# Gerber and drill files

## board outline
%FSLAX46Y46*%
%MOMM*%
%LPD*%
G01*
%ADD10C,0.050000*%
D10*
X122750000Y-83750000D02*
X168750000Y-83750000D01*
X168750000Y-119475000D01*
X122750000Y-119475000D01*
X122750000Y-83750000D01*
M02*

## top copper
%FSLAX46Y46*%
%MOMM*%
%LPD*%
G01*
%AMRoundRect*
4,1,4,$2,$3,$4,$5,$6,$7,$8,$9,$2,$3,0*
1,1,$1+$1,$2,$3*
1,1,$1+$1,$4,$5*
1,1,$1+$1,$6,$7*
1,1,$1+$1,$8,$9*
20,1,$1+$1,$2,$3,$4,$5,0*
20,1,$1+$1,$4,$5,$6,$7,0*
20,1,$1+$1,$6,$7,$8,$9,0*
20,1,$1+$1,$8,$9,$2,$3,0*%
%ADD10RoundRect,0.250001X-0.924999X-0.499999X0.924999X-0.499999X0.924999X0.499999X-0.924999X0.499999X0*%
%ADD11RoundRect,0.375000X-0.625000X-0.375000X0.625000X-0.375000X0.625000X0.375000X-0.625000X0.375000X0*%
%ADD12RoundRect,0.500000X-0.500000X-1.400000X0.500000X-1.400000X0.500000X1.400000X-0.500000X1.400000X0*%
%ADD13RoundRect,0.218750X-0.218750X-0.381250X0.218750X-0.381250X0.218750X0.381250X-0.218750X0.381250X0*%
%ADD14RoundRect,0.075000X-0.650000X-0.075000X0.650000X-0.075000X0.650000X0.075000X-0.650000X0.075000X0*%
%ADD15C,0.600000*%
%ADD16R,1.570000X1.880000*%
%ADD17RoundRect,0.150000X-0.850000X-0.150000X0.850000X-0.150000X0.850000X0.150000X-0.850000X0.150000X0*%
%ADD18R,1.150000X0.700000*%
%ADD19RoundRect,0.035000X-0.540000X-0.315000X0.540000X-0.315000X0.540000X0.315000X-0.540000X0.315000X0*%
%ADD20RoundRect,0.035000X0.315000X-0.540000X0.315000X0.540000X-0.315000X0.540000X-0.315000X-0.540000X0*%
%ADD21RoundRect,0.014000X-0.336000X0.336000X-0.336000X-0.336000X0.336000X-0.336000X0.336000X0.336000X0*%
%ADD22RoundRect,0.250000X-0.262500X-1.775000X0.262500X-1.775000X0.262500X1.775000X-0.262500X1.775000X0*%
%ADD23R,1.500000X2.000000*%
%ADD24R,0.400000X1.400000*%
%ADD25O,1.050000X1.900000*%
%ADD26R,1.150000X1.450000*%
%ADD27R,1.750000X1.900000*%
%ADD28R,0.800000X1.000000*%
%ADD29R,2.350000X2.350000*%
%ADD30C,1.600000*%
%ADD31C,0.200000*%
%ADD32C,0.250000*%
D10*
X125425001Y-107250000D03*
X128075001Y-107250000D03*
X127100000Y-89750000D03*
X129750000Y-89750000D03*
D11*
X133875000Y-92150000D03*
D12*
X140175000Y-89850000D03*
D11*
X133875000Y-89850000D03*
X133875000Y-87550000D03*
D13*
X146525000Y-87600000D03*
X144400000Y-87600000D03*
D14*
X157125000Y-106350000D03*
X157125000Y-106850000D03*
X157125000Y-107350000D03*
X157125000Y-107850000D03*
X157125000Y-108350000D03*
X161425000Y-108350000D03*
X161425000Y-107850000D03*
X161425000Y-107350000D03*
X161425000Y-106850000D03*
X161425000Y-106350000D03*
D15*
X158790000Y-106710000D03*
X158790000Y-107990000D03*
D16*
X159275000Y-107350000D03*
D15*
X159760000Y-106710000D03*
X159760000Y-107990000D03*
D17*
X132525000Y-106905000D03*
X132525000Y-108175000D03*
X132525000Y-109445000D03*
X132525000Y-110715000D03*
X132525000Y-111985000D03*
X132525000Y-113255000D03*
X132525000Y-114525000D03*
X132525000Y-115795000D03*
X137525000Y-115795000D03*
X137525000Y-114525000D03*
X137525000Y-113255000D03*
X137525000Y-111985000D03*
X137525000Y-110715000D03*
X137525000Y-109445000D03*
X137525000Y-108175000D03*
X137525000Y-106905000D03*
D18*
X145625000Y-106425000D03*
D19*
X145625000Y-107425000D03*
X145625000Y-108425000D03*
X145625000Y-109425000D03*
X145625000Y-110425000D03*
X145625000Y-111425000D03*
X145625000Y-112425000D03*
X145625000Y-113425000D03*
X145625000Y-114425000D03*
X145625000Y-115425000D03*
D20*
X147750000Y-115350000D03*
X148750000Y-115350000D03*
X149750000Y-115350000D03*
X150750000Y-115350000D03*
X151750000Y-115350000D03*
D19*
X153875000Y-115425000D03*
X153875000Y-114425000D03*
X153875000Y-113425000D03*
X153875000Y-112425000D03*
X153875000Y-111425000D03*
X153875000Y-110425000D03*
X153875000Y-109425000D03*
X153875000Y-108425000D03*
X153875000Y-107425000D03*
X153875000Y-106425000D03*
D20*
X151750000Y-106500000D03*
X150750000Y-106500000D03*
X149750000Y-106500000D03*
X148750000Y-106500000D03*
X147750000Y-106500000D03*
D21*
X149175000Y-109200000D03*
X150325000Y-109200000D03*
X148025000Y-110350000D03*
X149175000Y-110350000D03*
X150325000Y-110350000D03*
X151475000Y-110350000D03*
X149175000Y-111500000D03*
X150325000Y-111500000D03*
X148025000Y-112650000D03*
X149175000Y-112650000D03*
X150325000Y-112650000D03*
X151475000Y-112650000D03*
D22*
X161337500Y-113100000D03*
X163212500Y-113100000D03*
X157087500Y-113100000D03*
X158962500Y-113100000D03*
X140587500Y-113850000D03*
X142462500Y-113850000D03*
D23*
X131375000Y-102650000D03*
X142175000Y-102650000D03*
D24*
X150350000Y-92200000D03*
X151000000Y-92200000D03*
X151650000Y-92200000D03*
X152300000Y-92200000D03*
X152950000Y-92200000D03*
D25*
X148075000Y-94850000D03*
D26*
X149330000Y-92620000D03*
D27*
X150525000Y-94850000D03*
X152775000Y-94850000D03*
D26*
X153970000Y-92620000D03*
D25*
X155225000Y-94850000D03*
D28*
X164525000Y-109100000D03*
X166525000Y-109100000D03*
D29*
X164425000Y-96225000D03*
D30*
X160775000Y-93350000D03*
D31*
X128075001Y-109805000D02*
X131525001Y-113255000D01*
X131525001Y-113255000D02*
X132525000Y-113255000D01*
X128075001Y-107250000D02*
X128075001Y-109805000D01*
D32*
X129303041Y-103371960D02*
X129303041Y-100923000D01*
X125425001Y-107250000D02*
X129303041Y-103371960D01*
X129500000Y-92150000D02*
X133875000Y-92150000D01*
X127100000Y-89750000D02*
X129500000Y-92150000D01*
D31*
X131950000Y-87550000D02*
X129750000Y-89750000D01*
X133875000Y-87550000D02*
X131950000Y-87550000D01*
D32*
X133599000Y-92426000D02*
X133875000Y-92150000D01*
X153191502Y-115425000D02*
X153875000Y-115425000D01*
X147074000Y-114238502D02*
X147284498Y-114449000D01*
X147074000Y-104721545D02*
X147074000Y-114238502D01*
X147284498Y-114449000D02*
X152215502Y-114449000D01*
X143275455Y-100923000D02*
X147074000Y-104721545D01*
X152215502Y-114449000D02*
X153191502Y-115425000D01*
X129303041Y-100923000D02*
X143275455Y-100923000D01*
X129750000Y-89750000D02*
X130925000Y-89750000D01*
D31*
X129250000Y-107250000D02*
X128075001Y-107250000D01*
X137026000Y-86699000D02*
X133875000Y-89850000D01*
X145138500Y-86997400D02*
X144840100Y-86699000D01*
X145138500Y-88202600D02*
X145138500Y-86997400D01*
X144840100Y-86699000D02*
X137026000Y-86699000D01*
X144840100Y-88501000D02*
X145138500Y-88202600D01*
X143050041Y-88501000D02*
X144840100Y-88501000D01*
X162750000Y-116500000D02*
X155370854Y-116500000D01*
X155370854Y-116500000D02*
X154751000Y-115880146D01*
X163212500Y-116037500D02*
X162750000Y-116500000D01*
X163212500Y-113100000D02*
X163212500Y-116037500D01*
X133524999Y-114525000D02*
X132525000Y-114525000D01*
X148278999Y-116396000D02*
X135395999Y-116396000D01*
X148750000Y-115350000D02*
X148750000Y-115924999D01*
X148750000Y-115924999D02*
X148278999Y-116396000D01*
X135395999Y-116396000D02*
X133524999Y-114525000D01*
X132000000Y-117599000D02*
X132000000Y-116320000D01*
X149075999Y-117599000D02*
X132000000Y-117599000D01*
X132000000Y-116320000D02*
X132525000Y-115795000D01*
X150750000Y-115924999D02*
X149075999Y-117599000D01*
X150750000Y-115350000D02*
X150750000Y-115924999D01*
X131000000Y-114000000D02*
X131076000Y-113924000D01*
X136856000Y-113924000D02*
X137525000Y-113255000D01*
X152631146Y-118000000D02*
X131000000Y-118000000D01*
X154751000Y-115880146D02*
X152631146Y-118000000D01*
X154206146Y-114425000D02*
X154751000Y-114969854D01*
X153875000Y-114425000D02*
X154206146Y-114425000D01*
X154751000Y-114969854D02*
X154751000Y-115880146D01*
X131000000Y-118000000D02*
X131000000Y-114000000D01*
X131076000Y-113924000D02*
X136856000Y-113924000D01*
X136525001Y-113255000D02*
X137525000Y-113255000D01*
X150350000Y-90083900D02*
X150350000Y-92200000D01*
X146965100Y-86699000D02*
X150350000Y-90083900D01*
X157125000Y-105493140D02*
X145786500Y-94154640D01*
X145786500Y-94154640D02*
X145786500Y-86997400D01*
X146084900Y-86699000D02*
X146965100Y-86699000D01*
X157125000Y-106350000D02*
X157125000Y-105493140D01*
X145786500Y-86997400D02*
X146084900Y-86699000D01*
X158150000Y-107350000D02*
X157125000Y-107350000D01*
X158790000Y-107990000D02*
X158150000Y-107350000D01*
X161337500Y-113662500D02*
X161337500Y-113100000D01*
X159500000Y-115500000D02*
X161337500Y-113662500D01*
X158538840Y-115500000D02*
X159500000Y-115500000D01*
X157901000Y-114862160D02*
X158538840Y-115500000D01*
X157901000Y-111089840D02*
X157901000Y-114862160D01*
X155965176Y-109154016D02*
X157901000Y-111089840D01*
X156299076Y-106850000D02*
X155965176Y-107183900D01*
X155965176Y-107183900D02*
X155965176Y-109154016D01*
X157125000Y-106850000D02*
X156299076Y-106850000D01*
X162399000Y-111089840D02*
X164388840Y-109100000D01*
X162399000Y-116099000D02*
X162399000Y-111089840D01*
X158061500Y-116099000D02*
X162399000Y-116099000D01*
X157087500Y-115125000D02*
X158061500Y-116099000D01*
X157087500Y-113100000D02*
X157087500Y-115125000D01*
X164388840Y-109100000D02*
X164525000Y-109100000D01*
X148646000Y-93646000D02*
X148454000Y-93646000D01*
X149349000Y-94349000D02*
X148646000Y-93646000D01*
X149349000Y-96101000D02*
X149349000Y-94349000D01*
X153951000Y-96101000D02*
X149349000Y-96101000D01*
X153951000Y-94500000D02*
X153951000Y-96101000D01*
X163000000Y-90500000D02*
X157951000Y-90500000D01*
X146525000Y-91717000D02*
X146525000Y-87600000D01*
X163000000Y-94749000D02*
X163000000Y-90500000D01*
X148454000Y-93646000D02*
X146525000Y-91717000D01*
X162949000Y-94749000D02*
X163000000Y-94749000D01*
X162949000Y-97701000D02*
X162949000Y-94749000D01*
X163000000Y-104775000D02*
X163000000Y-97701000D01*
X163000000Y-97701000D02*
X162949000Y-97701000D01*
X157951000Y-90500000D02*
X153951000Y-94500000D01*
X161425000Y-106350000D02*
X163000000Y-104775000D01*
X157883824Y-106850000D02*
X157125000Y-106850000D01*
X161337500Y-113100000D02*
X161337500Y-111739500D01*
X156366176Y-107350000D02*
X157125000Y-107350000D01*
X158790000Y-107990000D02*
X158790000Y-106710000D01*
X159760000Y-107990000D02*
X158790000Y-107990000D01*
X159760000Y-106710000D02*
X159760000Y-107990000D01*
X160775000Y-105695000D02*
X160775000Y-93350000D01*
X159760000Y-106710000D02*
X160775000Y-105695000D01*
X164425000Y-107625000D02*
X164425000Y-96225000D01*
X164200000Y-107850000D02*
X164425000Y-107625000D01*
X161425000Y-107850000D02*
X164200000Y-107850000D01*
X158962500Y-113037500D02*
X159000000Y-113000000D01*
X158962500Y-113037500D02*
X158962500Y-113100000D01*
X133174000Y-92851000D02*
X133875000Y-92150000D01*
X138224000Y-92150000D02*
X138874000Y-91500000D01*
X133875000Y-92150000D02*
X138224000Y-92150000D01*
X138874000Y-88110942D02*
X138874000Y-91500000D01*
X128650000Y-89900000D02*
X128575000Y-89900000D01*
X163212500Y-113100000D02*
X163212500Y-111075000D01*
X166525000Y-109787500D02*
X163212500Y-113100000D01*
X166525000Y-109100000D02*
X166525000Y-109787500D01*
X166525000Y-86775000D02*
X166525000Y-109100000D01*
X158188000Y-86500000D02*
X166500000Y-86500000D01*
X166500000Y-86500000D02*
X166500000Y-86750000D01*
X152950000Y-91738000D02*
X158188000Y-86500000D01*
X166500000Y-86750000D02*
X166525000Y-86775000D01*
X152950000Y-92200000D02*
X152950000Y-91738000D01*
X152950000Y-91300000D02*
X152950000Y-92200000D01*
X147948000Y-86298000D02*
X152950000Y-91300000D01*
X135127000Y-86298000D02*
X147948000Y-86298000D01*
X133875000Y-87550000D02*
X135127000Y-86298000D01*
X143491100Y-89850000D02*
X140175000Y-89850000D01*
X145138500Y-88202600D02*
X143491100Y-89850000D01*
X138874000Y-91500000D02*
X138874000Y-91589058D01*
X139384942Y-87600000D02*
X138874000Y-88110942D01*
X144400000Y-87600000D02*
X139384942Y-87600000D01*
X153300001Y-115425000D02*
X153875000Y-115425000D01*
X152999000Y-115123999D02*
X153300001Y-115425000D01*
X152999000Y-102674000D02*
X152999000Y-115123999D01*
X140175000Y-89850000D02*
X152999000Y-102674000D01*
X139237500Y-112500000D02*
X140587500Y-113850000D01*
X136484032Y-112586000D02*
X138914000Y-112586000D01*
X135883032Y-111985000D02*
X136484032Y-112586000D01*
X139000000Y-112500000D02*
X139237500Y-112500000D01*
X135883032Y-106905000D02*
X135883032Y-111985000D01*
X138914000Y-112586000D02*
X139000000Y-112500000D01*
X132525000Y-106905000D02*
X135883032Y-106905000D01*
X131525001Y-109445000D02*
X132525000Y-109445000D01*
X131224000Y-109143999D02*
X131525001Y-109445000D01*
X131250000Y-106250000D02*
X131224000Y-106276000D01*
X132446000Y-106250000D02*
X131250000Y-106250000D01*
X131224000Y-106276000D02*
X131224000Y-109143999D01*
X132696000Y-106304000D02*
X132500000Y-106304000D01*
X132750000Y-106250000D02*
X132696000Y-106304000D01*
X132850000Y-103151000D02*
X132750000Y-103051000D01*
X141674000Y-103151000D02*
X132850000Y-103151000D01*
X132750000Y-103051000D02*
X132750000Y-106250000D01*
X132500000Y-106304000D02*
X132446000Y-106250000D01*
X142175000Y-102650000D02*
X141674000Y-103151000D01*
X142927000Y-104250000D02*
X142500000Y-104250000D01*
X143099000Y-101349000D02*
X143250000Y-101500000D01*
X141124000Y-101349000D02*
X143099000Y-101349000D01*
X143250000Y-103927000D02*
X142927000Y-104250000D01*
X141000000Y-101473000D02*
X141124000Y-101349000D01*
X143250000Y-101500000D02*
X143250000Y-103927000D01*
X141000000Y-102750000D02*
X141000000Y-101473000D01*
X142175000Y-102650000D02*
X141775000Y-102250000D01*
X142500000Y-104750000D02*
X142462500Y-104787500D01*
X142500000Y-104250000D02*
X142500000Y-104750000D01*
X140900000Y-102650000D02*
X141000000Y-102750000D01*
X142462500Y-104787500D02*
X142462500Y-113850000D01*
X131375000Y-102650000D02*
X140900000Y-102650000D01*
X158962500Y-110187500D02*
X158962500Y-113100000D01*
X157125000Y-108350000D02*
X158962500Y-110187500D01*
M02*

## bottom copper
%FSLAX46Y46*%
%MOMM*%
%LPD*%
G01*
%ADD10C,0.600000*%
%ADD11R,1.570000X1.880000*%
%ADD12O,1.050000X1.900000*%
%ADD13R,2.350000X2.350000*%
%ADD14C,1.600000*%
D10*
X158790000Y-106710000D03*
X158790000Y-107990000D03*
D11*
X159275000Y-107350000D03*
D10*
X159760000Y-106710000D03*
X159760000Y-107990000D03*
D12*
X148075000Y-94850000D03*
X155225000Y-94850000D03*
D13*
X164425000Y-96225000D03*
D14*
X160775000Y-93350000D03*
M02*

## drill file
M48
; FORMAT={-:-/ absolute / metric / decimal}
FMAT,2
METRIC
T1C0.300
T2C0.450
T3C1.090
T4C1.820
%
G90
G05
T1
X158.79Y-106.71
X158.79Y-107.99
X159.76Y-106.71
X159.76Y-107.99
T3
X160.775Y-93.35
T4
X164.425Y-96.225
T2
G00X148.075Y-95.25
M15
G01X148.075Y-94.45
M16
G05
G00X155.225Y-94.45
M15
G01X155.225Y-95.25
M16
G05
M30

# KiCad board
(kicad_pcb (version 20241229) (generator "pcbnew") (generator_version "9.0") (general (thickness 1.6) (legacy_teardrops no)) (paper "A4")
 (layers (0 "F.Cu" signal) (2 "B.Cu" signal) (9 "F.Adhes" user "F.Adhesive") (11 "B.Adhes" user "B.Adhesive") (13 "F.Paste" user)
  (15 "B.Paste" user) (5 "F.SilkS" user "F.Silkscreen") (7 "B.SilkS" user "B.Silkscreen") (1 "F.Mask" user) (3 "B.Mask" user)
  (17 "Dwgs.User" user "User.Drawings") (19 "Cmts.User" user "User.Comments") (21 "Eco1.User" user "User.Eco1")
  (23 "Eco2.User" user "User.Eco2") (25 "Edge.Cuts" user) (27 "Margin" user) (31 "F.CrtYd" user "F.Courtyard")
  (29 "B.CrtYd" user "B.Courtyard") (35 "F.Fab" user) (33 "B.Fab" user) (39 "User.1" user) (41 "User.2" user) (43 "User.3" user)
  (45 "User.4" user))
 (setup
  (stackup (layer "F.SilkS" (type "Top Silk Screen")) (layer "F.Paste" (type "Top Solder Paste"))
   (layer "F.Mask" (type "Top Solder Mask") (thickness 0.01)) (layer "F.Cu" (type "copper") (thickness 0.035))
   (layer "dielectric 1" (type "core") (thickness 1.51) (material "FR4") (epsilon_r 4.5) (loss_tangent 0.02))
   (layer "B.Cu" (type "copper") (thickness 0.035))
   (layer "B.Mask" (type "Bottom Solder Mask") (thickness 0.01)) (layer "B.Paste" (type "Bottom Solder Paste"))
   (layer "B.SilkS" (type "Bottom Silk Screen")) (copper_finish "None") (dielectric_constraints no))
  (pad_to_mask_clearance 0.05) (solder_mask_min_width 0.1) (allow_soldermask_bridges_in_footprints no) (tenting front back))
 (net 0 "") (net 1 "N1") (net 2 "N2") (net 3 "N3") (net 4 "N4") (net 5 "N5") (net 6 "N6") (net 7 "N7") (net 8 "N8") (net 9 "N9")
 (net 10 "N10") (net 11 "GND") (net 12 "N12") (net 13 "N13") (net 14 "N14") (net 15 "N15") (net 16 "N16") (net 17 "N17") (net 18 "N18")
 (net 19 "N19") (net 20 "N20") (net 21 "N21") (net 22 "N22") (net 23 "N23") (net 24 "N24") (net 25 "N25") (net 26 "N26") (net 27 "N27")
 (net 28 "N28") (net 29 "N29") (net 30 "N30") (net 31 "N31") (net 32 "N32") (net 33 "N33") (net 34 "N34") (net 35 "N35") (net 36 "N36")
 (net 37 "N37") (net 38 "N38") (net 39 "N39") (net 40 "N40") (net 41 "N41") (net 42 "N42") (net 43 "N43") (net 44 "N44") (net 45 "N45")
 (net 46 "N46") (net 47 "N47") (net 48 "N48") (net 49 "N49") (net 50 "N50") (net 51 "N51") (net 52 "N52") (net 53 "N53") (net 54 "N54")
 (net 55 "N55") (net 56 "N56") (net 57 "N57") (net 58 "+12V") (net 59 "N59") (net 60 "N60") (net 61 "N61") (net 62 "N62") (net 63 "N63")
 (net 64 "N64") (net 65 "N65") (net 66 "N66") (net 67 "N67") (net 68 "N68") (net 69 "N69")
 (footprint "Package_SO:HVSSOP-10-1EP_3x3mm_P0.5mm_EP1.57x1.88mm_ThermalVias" (layer "F.Cu") (at 159.275 107.35)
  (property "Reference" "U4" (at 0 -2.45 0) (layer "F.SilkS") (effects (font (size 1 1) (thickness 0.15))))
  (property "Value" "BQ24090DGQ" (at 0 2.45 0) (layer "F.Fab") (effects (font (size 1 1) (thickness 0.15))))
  (pad "" smd roundrect (at -0.39 -0.47) (size 0.63 0.76) (layers "F.Paste") (roundrect_rratio 0.25))
  (pad "" smd roundrect (at -0.39 0.47) (size 0.63 0.76) (layers "F.Paste") (roundrect_rratio 0.25))
  (pad "" smd roundrect (at 0.39 -0.47) (size 0.63 0.76) (layers "F.Paste") (roundrect_rratio 0.25))
  (pad "" smd roundrect (at 0.39 0.47) (size 0.63 0.76) (layers "F.Paste") (roundrect_rratio 0.25))
  (pad "1" smd roundrect (at -2.15 -1) (size 1.45 0.3) (layers "F.Cu" "F.Mask" "F.Paste") (roundrect_rratio 0.25) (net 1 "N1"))
  (pad "2" smd roundrect (at -2.15 -0.5) (size 1.45 0.3) (layers "F.Cu" "F.Mask" "F.Paste") (roundrect_rratio 0.25) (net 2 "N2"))
  (pad "3" smd roundrect (at -2.15 0) (size 1.45 0.3) (layers "F.Cu" "F.Mask" "F.Paste") (roundrect_rratio 0.25) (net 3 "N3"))
  (pad "4" smd roundrect (at -2.15 0.5) (size 1.45 0.3) (layers "F.Cu" "F.Mask" "F.Paste") (roundrect_rratio 0.25) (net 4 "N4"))
  (pad "5" smd roundrect (at -2.15 1) (size 1.45 0.3) (layers "F.Cu" "F.Mask" "F.Paste") (roundrect_rratio 0.25) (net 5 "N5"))
  (pad "6" smd roundrect (at 2.15 1) (size 1.45 0.3) (layers "F.Cu" "F.Mask" "F.Paste") (roundrect_rratio 0.25) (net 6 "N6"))
  (pad "7" smd roundrect (at 2.15 0.5) (size 1.45 0.3) (layers "F.Cu" "F.Mask" "F.Paste") (roundrect_rratio 0.25) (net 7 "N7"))
  (pad "8" smd roundrect (at 2.15 0) (size 1.45 0.3) (layers "F.Cu" "F.Mask" "F.Paste") (roundrect_rratio 0.25) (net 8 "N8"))
  (pad "9" smd roundrect (at 2.15 -0.5) (size 1.45 0.3) (layers "F.Cu" "F.Mask" "F.Paste") (roundrect_rratio 0.25) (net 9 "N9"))
  (pad "10" smd roundrect (at 2.15 -1) (size 1.45 0.3) (layers "F.Cu" "F.Mask" "F.Paste") (roundrect_rratio 0.25) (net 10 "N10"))
  (pad "11" thru_hole circle (at -0.485 -0.64) (size 0.6 0.6) (drill 0.3) (layers "*.Cu") (remove_unused_layers no) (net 3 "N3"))
  (pad "11" thru_hole circle (at -0.485 0.64) (size 0.6 0.6) (drill 0.3) (layers "*.Cu") (remove_unused_layers no) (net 3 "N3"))
  (pad "11" smd rect (at 0 0) (size 1.57 1.88) (layers "F.Cu" "F.Mask") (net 3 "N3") (zone_connect 2))
  (pad "11" smd rect (at 0 0) (size 1.57 1.88) (layers "B.Cu") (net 3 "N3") (zone_connect 2))
  (pad "11" thru_hole circle (at 0.485 -0.64) (size 0.6 0.6) (drill 0.3) (layers "*.Cu") (remove_unused_layers no) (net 3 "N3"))
  (pad "11" thru_hole circle (at 0.485 0.64) (size 0.6 0.6) (drill 0.3) (layers "*.Cu") (remove_unused_layers no) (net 3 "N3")))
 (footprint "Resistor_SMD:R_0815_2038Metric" (layer "F.Cu") (at 162.275 113.1)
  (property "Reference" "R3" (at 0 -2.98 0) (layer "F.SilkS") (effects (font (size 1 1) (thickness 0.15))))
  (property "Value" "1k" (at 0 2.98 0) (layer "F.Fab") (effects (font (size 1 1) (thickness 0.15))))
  (pad "1" smd roundrect (at -0.9375 0) (size 1.025 4.05) (layers "F.Cu" "F.Mask" "F.Paste") (roundrect_rratio 0.243902) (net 2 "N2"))
  (pad "2" smd roundrect (at 0.9375 0) (size 1.025 4.05) (layers "F.Cu" "F.Mask" "F.Paste") (roundrect_rratio 0.243902) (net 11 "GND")))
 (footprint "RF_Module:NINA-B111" (layer "F.Cu") (at 149.75 110.925)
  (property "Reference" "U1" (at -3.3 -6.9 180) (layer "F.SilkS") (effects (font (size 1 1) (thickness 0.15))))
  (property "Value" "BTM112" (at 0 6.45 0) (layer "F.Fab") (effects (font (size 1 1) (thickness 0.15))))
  (pad "1" smd rect (at -4.125 -4.5) (size 1.15 0.7) (layers "F.Cu" "F.Mask" "F.Paste") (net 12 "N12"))
  (pad "2" smd roundrect (at -4.125 -3.5) (size 1.15 0.7) (layers "F.Cu" "F.Mask" "F.Paste") (roundrect_rratio 0.05) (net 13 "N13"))
  (pad "3" smd roundrect (at -4.125 -2.5) (size 1.15 0.7) (layers "F.Cu" "F.Mask" "F.Paste") (roundrect_rratio 0.05) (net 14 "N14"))
  (pad "4" smd roundrect (at -4.125 -1.5) (size 1.15 0.7) (layers "F.Cu" "F.Mask" "F.Paste") (roundrect_rratio 0.05) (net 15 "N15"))
  (pad "5" smd roundrect (at -4.125 -0.5) (size 1.15 0.7) (layers "F.Cu" "F.Mask" "F.Paste") (roundrect_rratio 0.05) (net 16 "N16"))
  (pad "6" smd roundrect (at -4.125 0.5) (size 1.15 0.7) (layers "F.Cu" "F.Mask" "F.Paste") (roundrect_rratio 0.05) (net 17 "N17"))
  (pad "7" smd roundrect (at -4.125 1.5) (size 1.15 0.7) (layers "F.Cu" "F.Mask" "F.Paste") (roundrect_rratio 0.05) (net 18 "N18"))
  (pad "8" smd roundrect (at -4.125 2.5) (size 1.15 0.7) (layers "F.Cu" "F.Mask" "F.Paste") (roundrect_rratio 0.05) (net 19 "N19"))
  (pad "9" smd roundrect (at -4.125 3.5) (size 1.15 0.7) (layers "F.Cu" "F.Mask" "F.Paste") (roundrect_rratio 0.05) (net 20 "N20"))
  (pad "10" smd roundrect (at -4.125 4.5) (size 1.15 0.7) (layers "F.Cu" "F.Mask" "F.Paste") (roundrect_rratio 0.05) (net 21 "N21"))
  (pad "11" smd roundrect (at -2 4.425 90) (size 1.15 0.7) (layers "F.Cu" "F.Mask" "F.Paste") (roundrect_rratio 0.05) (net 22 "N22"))
  (pad "12" smd roundrect (at -1 4.425 90) (size 1.15 0.7) (layers "F.Cu" "F.Mask" "F.Paste") (roundrect_rratio 0.05) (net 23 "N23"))
  (pad "13" smd roundrect (at 0 4.425 90) (size 1.15 0.7) (layers "F.Cu" "F.Mask" "F.Paste") (roundrect_rratio 0.05) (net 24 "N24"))
  (pad "14" smd roundrect (at 1 4.425 90) (size 1.15 0.7) (layers "F.Cu" "F.Mask" "F.Paste") (roundrect_rratio 0.05) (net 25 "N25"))
  (pad "15" smd roundrect (at 2 4.425 90) (size 1.15 0.7) (layers "F.Cu" "F.Mask" "F.Paste") (roundrect_rratio 0.05) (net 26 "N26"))
  (pad "16" smd roundrect (at 4.125 4.5) (size 1.15 0.7) (layers "F.Cu" "F.Mask" "F.Paste") (roundrect_rratio 0.05) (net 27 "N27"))
  (pad "17" smd roundrect (at 4.125 3.5) (size 1.15 0.7) (layers "F.Cu" "F.Mask" "F.Paste") (roundrect_rratio 0.05) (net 11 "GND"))
  (pad "18" smd roundrect (at 4.125 2.5) (size 1.15 0.7) (layers "F.Cu" "F.Mask" "F.Paste") (roundrect_rratio 0.05) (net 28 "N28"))
  (pad "19" smd roundrect (at 4.125 1.5) (size 1.15 0.7) (layers "F.Cu" "F.Mask" "F.Paste") (roundrect_rratio 0.05) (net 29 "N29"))
  (pad "20" smd roundrect (at 4.125 0.5) (size 1.15 0.7) (layers "F.Cu" "F.Mask" "F.Paste") (roundrect_rratio 0.05) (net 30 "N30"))
  (pad "21" smd roundrect (at 4.125 -0.5) (size 1.15 0.7) (layers "F.Cu" "F.Mask" "F.Paste") (roundrect_rratio 0.05) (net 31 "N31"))
  (pad "22" smd roundrect (at 4.125 -1.5) (size 1.15 0.7) (layers "F.Cu" "F.Mask" "F.Paste") (roundrect_rratio 0.05) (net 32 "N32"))
  (pad "23" smd roundrect (at 4.125 -2.5) (size 1.15 0.7) (layers "F.Cu" "F.Mask" "F.Paste") (roundrect_rratio 0.05) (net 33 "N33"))
  (pad "24" smd roundrect (at 4.125 -3.5) (size 1.15 0.7) (layers "F.Cu" "F.Mask" "F.Paste") (roundrect_rratio 0.05) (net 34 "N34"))
  (pad "25" smd roundrect (at 4.125 -4.5) (size 1.15 0.7) (layers "F.Cu" "F.Mask" "F.Paste") (roundrect_rratio 0.05) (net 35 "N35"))
  (pad "26" smd roundrect (at 2 -4.425 90) (size 1.15 0.7) (layers "F.Cu" "F.Mask" "F.Paste") (roundrect_rratio 0.05) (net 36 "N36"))
  (pad "27" smd roundrect (at 1 -4.425 90) (size 1.15 0.7) (layers "F.Cu" "F.Mask" "F.Paste") (roundrect_rratio 0.05) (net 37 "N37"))
  (pad "28" smd roundrect (at 0 -4.425 90) (size 1.15 0.7) (layers "F.Cu" "F.Mask" "F.Paste") (roundrect_rratio 0.05) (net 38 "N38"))
  (pad "29" smd roundrect (at -1 -4.425 90) (size 1.15 0.7) (layers "F.Cu" "F.Mask" "F.Paste") (roundrect_rratio 0.05) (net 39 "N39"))
  (pad "30" smd roundrect (at -2 -4.425 90) (size 1.15 0.7) (layers "F.Cu" "F.Mask" "F.Paste") (roundrect_rratio 0.05) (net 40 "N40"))
  (pad "31" smd roundrect (at -0.575 -1.725 270) (size 0.7 0.7) (layers "F.Cu" "F.Mask" "F.Paste") (roundrect_rratio 0.02) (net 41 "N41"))
  (pad "32" smd roundrect (at 0.575 -1.725 270) (size 0.7 0.7) (layers "F.Cu" "F.Mask" "F.Paste") (roundrect_rratio 0.02) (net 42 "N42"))
  (pad "33" smd roundrect (at -1.725 -0.575 270) (size 0.7 0.7) (layers "F.Cu" "F.Mask" "F.Paste") (roundrect_rratio 0.02) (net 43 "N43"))
  (pad "34" smd roundrect (at -0.575 -0.575 270) (size 0.7 0.7) (layers "F.Cu" "F.Mask" "F.Paste") (roundrect_rratio 0.02) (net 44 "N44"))
  (pad "35" smd roundrect (at 0.575 -0.575 270) (size 0.7 0.7) (layers "F.Cu" "F.Mask" "F.Paste") (roundrect_rratio 0.02))
  (pad "36" smd roundrect (at 1.725 -0.575 270) (size 0.7 0.7) (layers "F.Cu" "F.Mask" "F.Paste") (roundrect_rratio 0.02))
  (pad "37" smd roundrect (at -0.575 0.575 270) (size 0.7 0.7) (layers "F.Cu" "F.Mask" "F.Paste") (roundrect_rratio 0.02))
  (pad "38" smd roundrect (at 0.575 0.575 270) (size 0.7 0.7) (layers "F.Cu" "F.Mask" "F.Paste") (roundrect_rratio 0.02))
  (pad "39" smd roundrect (at -1.725 1.725 270) (size 0.7 0.7) (layers "F.Cu" "F.Mask" "F.Paste") (roundrect_rratio 0.02))
  (pad "40" smd roundrect (at -0.575 1.725 270) (size 0.7 0.7) (layers "F.Cu" "F.Mask" "F.Paste") (roundrect_rratio 0.02))
  (pad "41" smd roundrect (at 0.575 1.725 270) (size 0.7 0.7) (layers "F.Cu" "F.Mask" "F.Paste") (roundrect_rratio 0.02))
  (pad "42" smd roundrect (at 1.725 1.725 270) (size 0.7 0.7) (layers "F.Cu" "F.Mask" "F.Paste") (roundrect_rratio 0.02))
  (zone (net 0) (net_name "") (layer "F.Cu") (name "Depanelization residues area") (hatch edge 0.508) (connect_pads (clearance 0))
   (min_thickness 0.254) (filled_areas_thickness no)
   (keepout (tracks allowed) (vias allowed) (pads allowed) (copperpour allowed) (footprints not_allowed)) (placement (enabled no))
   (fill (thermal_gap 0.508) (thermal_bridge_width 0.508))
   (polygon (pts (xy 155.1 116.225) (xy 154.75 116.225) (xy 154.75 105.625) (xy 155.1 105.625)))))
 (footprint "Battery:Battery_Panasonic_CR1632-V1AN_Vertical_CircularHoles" (layer "F.Cu") (at 164.425 96.225 90)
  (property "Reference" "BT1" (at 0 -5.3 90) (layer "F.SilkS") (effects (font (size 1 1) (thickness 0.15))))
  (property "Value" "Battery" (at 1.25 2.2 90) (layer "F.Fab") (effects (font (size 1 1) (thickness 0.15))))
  (pad "1" thru_hole rect (at 0 0 180) (size 2.35 2.35) (drill 1.82) (layers "*.Cu" "*.Mask") (remove_unused_layers no) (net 7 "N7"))
  (pad "2" thru_hole circle (at 2.875 -3.65 90) (size 1.6 1.6) (drill 1.09) (layers "*.Cu" "*.Mask") (remove_unused_layers no) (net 3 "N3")))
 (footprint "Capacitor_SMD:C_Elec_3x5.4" (layer "F.Cu") (at 126.750001 107.25)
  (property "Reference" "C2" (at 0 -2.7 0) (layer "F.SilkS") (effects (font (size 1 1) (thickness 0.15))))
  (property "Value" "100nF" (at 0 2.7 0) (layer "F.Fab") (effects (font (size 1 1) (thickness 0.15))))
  (pad "1" smd roundrect (at -1.325 0) (size 2.35 1.5) (layers "F.Cu" "F.Mask" "F.Paste") (roundrect_rratio 0.166667) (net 27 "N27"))
  (pad "2" smd roundrect (at 1.325 0) (size 2.35 1.5) (layers "F.Cu" "F.Mask" "F.Paste") (roundrect_rratio 0.166667) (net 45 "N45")))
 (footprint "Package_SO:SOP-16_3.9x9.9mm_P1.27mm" (layer "F.Cu") (at 135.025 111.35)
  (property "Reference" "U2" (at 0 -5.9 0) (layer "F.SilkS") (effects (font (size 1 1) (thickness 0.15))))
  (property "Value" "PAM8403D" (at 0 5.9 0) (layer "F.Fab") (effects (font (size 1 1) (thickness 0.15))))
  (pad "1" smd roundrect (at -2.5 -4.445) (size 2 0.6) (layers "F.Cu" "F.Mask" "F.Paste") (roundrect_rratio 0.25) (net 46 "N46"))
  (pad "2" smd roundrect (at -2.5 -3.175) (size 2 0.6) (layers "F.Cu" "F.Mask" "F.Paste") (roundrect_rratio 0.25) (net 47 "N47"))
  (pad "3" smd roundrect (at -2.5 -1.905) (size 2 0.6) (layers "F.Cu" "F.Mask" "F.Paste") (roundrect_rratio 0.25) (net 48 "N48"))
  (pad "4" smd roundrect (at -2.5 -0.635) (size 2 0.6) (layers "F.Cu" "F.Mask" "F.Paste") (roundrect_rratio 0.25) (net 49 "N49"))
  (pad "5" smd roundrect (at -2.5 0.635) (size 2 0.6) (layers "F.Cu" "F.Mask" "F.Paste") (roundrect_rratio 0.25) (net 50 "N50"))
  (pad "6" smd roundrect (at -2.5 1.905) (size 2 0.6) (layers "F.Cu" "F.Mask" "F.Paste") (roundrect_rratio 0.25) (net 45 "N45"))
  (pad "7" smd roundrect (at -2.5 3.175) (size 2 0.6) (layers "F.Cu" "F.Mask" "F.Paste") (roundrect_rratio 0.25) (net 23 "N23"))
  (pad "8" smd roundrect (at -2.5 4.445) (size 2 0.6) (layers "F.Cu" "F.Mask" "F.Paste") (roundrect_rratio 0.25) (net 25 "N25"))
  (pad "9" smd roundrect (at 2.5 4.445) (size 2 0.6) (layers "F.Cu" "F.Mask" "F.Paste") (roundrect_rratio 0.25) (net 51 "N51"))
  (pad "10" smd roundrect (at 2.5 3.175) (size 2 0.6) (layers "F.Cu" "F.Mask" "F.Paste") (roundrect_rratio 0.25) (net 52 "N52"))
  (pad "11" smd roundrect (at 2.5 1.905) (size 2 0.6) (layers "F.Cu" "F.Mask" "F.Paste") (roundrect_rratio 0.25) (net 11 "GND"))
  (pad "12" smd roundrect (at 2.5 0.635) (size 2 0.6) (layers "F.Cu" "F.Mask" "F.Paste") (roundrect_rratio 0.25) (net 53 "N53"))
  (pad "13" smd roundrect (at 2.5 -0.635) (size 2 0.6) (layers "F.Cu" "F.Mask" "F.Paste") (roundrect_rratio 0.25) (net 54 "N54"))
  (pad "14" smd roundrect (at 2.5 -1.905) (size 2 0.6) (layers "F.Cu" "F.Mask" "F.Paste") (roundrect_rratio 0.25) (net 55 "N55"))
  (pad "15" smd roundrect (at 2.5 -3.175) (size 2 0.6) (layers "F.Cu" "F.Mask" "F.Paste") (roundrect_rratio 0.25) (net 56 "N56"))
  (pad "16" smd roundrect (at 2.5 -4.445) (size 2 0.6) (layers "F.Cu" "F.Mask" "F.Paste") (roundrect_rratio 0.25) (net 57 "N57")))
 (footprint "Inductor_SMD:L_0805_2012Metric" (layer "F.Cu") (at 145.4625 87.6)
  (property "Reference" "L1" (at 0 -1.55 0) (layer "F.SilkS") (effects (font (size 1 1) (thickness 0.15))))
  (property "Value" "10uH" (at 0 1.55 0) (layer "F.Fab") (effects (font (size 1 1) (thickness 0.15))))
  (pad "1" smd roundrect (at -1.0625 0) (size 0.875 1.2) (layers "F.Cu" "F.Mask" "F.Paste") (roundrect_rratio 0.25) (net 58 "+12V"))
  (pad "2" smd roundrect (at 1.0625 0) (size 0.875 1.2) (layers "F.Cu" "F.Mask" "F.Paste") (roundrect_rratio 0.25) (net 10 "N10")))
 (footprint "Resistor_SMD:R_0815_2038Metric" (layer "F.Cu") (at 141.525 113.85)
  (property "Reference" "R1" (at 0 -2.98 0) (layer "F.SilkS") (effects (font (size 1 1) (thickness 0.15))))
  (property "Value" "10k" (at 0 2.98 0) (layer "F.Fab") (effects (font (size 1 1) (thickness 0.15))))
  (pad "1" smd roundrect (at -0.9375 0) (size 1.025 4.05) (layers "F.Cu" "F.Mask" "F.Paste") (roundrect_rratio 0.243902) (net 46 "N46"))
  (pad "2" smd roundrect (at 0.9375 0) (size 1.025 4.05) (layers "F.Cu" "F.Mask" "F.Paste") (roundrect_rratio 0.243902) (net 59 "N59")))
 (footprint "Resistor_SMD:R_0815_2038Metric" (layer "F.Cu") (at 158.025 113.1)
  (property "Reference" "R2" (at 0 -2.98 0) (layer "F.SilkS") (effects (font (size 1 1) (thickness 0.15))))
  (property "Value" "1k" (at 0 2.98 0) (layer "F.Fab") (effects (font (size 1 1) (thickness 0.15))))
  (pad "1" smd roundrect (at -0.9375 0) (size 1.025 4.05) (layers "F.Cu" "F.Mask" "F.Paste") (roundrect_rratio 0.243902) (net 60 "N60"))
  (pad "2" smd roundrect (at 0.9375 0) (size 1.025 4.05) (layers "F.Cu" "F.Mask" "F.Paste") (roundrect_rratio 0.243902) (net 5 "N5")))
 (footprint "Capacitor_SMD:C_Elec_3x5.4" (layer "F.Cu") (at 128.425 89.75)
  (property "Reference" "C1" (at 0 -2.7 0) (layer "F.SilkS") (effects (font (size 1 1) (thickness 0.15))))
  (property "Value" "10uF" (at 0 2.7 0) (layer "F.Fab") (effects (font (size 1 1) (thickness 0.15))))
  (pad "1" smd roundrect (at -1.325 0) (size 2.35 1.5) (layers "F.Cu" "F.Mask" "F.Paste") (roundrect_rratio 0.166667) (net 58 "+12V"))
  (pad "2" smd roundrect (at 1.325 0) (size 2.35 1.5) (layers "F.Cu" "F.Mask" "F.Paste") (roundrect_rratio 0.166667) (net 11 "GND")))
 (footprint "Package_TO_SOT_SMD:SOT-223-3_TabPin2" (layer "F.Cu") (at 137.025 89.85)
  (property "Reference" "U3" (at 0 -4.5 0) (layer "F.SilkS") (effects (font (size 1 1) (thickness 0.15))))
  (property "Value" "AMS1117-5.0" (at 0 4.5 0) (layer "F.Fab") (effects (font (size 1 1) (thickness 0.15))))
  (pad "1" smd roundrect (at -3.15 -2.3) (size 2 1.5) (layers "F.Cu" "F.Mask" "F.Paste") (roundrect_rratio 0.25) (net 11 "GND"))
  (pad "2" smd roundrect (at -3.15 0) (size 2 1.5) (layers "F.Cu" "F.Mask" "F.Paste") (roundrect_rratio 0.25) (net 27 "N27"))
  (pad "2" smd roundrect (at 3.15 0) (size 2 3.8) (layers "F.Cu" "F.Mask" "F.Paste") (roundrect_rratio 0.25) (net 27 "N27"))
  (pad "3" smd roundrect (at -3.15 2.3) (size 2 1.5) (layers "F.Cu" "F.Mask" "F.Paste") (roundrect_rratio 0.25) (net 58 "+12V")))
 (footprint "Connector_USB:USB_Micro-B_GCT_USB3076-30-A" (layer "F.Cu") (at 151.65 93.65)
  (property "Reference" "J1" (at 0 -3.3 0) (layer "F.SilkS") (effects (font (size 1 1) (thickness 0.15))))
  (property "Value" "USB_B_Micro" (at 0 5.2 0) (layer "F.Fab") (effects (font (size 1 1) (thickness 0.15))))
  (pad "1" smd rect (at -1.3 -1.45) (size 0.4 1.4) (layers "F.Cu" "F.Mask" "F.Paste") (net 1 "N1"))
  (pad "2" smd rect (at -0.65 -1.45) (size 0.4 1.4) (layers "F.Cu" "F.Mask" "F.Paste") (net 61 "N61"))
  (pad "3" smd rect (at 0 -1.45) (size 0.4 1.4) (layers "F.Cu" "F.Mask" "F.Paste") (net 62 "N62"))
  (pad "4" smd rect (at 0.65 -1.45) (size 0.4 1.4) (layers "F.Cu" "F.Mask" "F.Paste") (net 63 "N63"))
  (pad "5" smd rect (at 1.3 -1.45) (size 0.4 1.4) (layers "F.Cu" "F.Mask" "F.Paste") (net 11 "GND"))
  (pad "6" thru_hole oval (at -3.575 1.2 180) (size 1.05 1.9) (drill oval 0.45 1.25) (layers "*.Cu" "*.Mask") (remove_unused_layers no)
   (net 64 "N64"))
  (pad "6" smd rect (at -2.32 -1.03) (size 1.15 1.45) (layers "F.Cu" "F.Mask" "F.Paste") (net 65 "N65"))
  (pad "6" smd rect (at -1.125 1.2) (size 1.75 1.9) (layers "F.Cu" "F.Mask" "F.Paste") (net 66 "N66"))
  (pad "6" smd rect (at 1.125 1.2) (size 1.75 1.9) (layers "F.Cu" "F.Mask" "F.Paste") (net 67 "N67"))
  (pad "6" smd rect (at 2.32 -1.03) (size 1.15 1.45) (layers "F.Cu" "F.Mask" "F.Paste") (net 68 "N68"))
  (pad "6" thru_hole oval (at 3.575 1.2) (size 1.05 1.9) (drill oval 0.45 1.25) (layers "*.Cu" "*.Mask") (remove_unused_layers no)
   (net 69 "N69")))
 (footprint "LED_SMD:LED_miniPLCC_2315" (layer "F.Cu") (at 165.525 109.1)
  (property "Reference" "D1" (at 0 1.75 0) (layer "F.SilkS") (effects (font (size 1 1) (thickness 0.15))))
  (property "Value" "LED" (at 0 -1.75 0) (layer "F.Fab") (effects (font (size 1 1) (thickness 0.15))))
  (pad "1" smd rect (at -1 0 180) (size 0.8 1) (layers "F.Cu" "F.Mask" "F.Paste") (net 60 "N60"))
  (pad "2" smd rect (at 1 0 180) (size 0.8 1) (layers "F.Cu" "F.Mask" "F.Paste") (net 11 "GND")))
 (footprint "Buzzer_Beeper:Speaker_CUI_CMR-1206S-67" (layer "F.Cu") (at 136.775 100.35)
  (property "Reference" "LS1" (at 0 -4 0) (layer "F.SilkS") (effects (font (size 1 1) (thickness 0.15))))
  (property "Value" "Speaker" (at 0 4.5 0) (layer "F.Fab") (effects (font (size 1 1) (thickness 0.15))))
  (pad "1" smd rect (at -5.4 2.3 180) (size 1.5 2) (layers "F.Cu" "F.Mask") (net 59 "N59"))
  (pad "2" smd rect (at 5.4 2.3 180) (size 1.5 2) (layers "F.Cu" "F.Mask") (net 48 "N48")))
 (gr_rect (start 122.75 83.75) (end 168.75 119.475) (stroke (width 0.05) (type default)) (fill no) (layer "Edge.Cuts"))
 (segment (start 156.366176 107.35) (end 157.125 107.35) (width 0.2) (layer "F.Cu") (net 3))
 (segment (start 158.15 107.35) (end 157.125 107.35) (width 0.2) (layer "F.Cu") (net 3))
 (segment (start 159.76 107.99) (end 158.79 107.99) (width 0.2) (layer "F.Cu") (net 3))
 (segment (start 160.775 105.695) (end 160.775 93.35) (width 0.2) (layer "F.Cu") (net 3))
 (segment (start 158.79 107.99) (end 158.79 106.71) (width 0.2) (layer "F.Cu") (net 3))
 (segment (start 158.79 107.99) (end 158.15 107.35) (width 0.2) (layer "F.Cu") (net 3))
 (segment (start 159.76 106.71) (end 160.775 105.695) (width 0.2) (layer "F.Cu") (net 3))
 (segment (start 159.76 106.71) (end 159.76 107.99) (width 0.2) (layer "F.Cu") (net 3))
 (segment (start 164.425 107.625) (end 164.425 96.225) (width 0.2) (layer "F.Cu") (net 7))
 (segment (start 164.2 107.85) (end 164.425 107.625) (width 0.2) (layer "F.Cu") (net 7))
 (segment (start 161.425 107.85) (end 164.2 107.85) (width 0.2) (layer "F.Cu") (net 7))
 (segment (start 144.4 87.6) (end 139.384942 87.6) (width 0.2) (layer "F.Cu") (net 58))
 (segment (start 129.5 92.15) (end 133.875 92.15) (width 0.25) (layer "F.Cu") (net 58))
 (segment (start 139.384942 87.6) (end 138.874 88.110942) (width 0.2) (layer "F.Cu") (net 58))
 (segment (start 127.1 89.75) (end 129.5 92.15) (width 0.25) (layer "F.Cu") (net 58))
 (segment (start 138.874 88.110942) (end 138.874 91.5) (width 0.2) (layer "F.Cu") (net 58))
 (segment (start 133.174 92.851) (end 133.875 92.15) (width 0.2) (layer "F.Cu") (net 58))
 (segment (start 138.874 91.5) (end 138.874 91.589058) (width 0.2) (layer "F.Cu") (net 58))
 (segment (start 133.875 92.15) (end 138.224 92.15) (width 0.2) (layer "F.Cu") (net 58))
 (segment (start 133.599 92.426) (end 133.875 92.15) (width 0.25) (layer "F.Cu") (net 58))
 (segment (start 138.224 92.15) (end 138.874 91.5) (width 0.2) (layer "F.Cu") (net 58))
 (segment (start 131.076 113.924) (end 136.856 113.924) (width 0.2) (layer "F.Cu") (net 11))
 (segment (start 131 114) (end 131.076 113.924) (width 0.2) (layer "F.Cu") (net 11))
 (segment (start 133.875 87.55) (end 131.95 87.55) (width 0.2) (layer "F.Cu") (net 11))
 (segment (start 163.2125 113.1) (end 163.2125 116.0375) (width 0.2) (layer "F.Cu") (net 11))
 (segment (start 166.525 109.7875) (end 163.2125 113.1) (width 0.2) (layer "F.Cu") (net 11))
 (segment (start 166.525 109.1) (end 166.525 109.7875) (width 0.2) (layer "F.Cu") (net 11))
 (segment (start 136.856 113.924) (end 137.525 113.255) (width 0.2) (layer "F.Cu") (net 11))
 (segment (start 155.370854 116.5) (end 154.751 115.880146) (width 0.2) (layer "F.Cu") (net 11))
 (segment (start 152.95 91.738) (end 158.188 86.5) (width 0.2) (layer "F.Cu") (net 11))
 (segment (start 166.5 86.75) (end 166.525 86.775) (width 0.2) (layer "F.Cu") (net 11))
 (segment (start 133.875 87.55) (end 135.127 86.298) (width 0.2) (layer "F.Cu") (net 11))
 (segment (start 152.95 92.2) (end 152.95 91.738) (width 0.2) (layer "F.Cu") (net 11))
 (segment (start 163.2125 116.0375) (end 162.75 116.5) (width 0.2) (layer "F.Cu") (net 11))
 (segment (start 163.2125 113.1) (end 163.2125 111.075) (width 0.2) (layer "F.Cu") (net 11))
 (segment (start 166.525 86.775) (end 166.525 109.1) (width 0.2) (layer "F.Cu") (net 11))
 (segment (start 135.127 86.298) (end 147.948 86.298) (width 0.2) (layer "F.Cu") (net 11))
 (segment (start 162.75 116.5) (end 155.370854 116.5) (width 0.2) (layer "F.Cu") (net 11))
 (segment (start 158.188 86.5) (end 166.5 86.5) (width 0.2) (layer "F.Cu") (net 11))
 (segment (start 153.875 114.425) (end 154.206146 114.425) (width 0.2) (layer "F.Cu") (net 11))
 (segment (start 147.948 86.298) (end 152.95 91.3) (width 0.2) (layer "F.Cu") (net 11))
 (segment (start 154.751 115.880146) (end 152.631146 118) (width 0.2) (layer "F.Cu") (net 11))
 (segment (start 136.525001 113.255) (end 137.525 113.255) (width 0.2) (layer "F.Cu") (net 11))
 (segment (start 152.95 91.3) (end 152.95 92.2) (width 0.2) (layer "F.Cu") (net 11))
 (segment (start 128.65 89.9) (end 128.575 89.9) (width 0.2) (layer "F.Cu") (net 11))
 (segment (start 166.5 86.5) (end 166.5 86.75) (width 0.2) (layer "F.Cu") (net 11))
 (segment (start 131.95 87.55) (end 129.75 89.75) (width 0.2) (layer "F.Cu") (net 11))
 (segment (start 154.206146 114.425) (end 154.751 114.969854) (width 0.2) (layer "F.Cu") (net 11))
 (segment (start 129.75 89.75) (end 130.925 89.75) (width 0.25) (layer "F.Cu") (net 11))
 (segment (start 152.631146 118) (end 131 118) (width 0.2) (layer "F.Cu") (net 11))
 (segment (start 154.751 114.969854) (end 154.751 115.880146) (width 0.2) (layer "F.Cu") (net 11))
 (segment (start 131 118) (end 131 114) (width 0.2) (layer "F.Cu") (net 11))
 (segment (start 128.075001 107.25) (end 128.075001 109.805) (width 0.2) (layer "F.Cu") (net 45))
 (segment (start 131.525001 113.255) (end 132.525 113.255) (width 0.2) (layer "F.Cu") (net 45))
 (segment (start 128.075001 109.805) (end 131.525001 113.255) (width 0.2) (layer "F.Cu") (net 45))
 (segment (start 129.25 107.25) (end 128.075001 107.25) (width 0.2) (layer "F.Cu") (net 45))
 (segment (start 144.8401 86.699) (end 137.026 86.699) (width 0.2) (layer "F.Cu") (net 27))
 (segment (start 147.074 104.721545) (end 147.074 114.238502) (width 0.25) (layer "F.Cu") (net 27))
 (segment (start 125.425001 107.25) (end 129.303041 103.37196) (width 0.25) (layer "F.Cu") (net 27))
 (segment (start 153.300001 115.425) (end 153.875 115.425) (width 0.2) (layer "F.Cu") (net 27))
 (segment (start 140.175 89.85) (end 152.999 102.674) (width 0.2) (layer "F.Cu") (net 27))
 (segment (start 144.8401 88.501) (end 145.1385 88.2026) (width 0.2) (layer "F.Cu") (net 27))
 (segment (start 147.284498 114.449) (end 152.215502 114.449) (width 0.25) (layer "F.Cu") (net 27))
 (segment (start 137.026 86.699) (end 133.875 89.85) (width 0.2) (layer "F.Cu") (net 27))
 (segment (start 129.303041 103.37196) (end 129.303041 100.923) (width 0.25) (layer "F.Cu") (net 27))
 (segment (start 145.1385 88.2026) (end 145.1385 86.9974) (width 0.2) (layer "F.Cu") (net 27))
 (segment (start 143.4911 89.85) (end 140.175 89.85) (width 0.2) (layer "F.Cu") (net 27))
 (segment (start 143.050041 88.501) (end 144.8401 88.501) (width 0.2) (layer "F.Cu") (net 27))
 (segment (start 147.074 114.238502) (end 147.284498 114.449) (width 0.25) (layer "F.Cu") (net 27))
 (segment (start 129.303041 100.923) (end 143.275455 100.923) (width 0.25) (layer "F.Cu") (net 27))
 (segment (start 152.999 115.123999) (end 153.300001 115.425) (width 0.2) (layer "F.Cu") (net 27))
 (segment (start 145.1385 86.9974) (end 144.8401 86.699) (width 0.2) (layer "F.Cu") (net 27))
 (segment (start 153.191502 115.425) (end 153.875 115.425) (width 0.25) (layer "F.Cu") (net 27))
 (segment (start 152.999 102.674) (end 152.999 115.123999) (width 0.2) (layer "F.Cu") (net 27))
 (segment (start 145.1385 88.2026) (end 143.4911 89.85) (width 0.2) (layer "F.Cu") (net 27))
 (segment (start 143.275455 100.923) (end 147.074 104.721545) (width 0.25) (layer "F.Cu") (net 27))
 (segment (start 152.215502 114.449) (end 153.191502 115.425) (width 0.25) (layer "F.Cu") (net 27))
 (segment (start 157.0875 115.125) (end 158.0615 116.099) (width 0.2) (layer "F.Cu") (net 60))
 (segment (start 157.0875 113.1) (end 157.0875 115.125) (width 0.2) (layer "F.Cu") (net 60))
 (segment (start 158.0615 116.099) (end 162.399 116.099) (width 0.2) (layer "F.Cu") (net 60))
 (segment (start 162.399 111.08984) (end 164.38884 109.1) (width 0.2) (layer "F.Cu") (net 60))
 (segment (start 162.399 116.099) (end 162.399 111.08984) (width 0.2) (layer "F.Cu") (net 60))
 (segment (start 164.38884 109.1) (end 164.525 109.1) (width 0.2) (layer "F.Cu") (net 60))
 (segment (start 157.125 106.35) (end 157.125 105.49314) (width 0.2) (layer "F.Cu") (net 1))
 (segment (start 150.35 90.0839) (end 150.35 92.2) (width 0.2) (layer "F.Cu") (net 1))
 (segment (start 145.7865 94.15464) (end 145.7865 86.9974) (width 0.2) (layer "F.Cu") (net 1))
 (segment (start 145.7865 86.9974) (end 146.0849 86.699) (width 0.2) (layer "F.Cu") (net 1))
 (segment (start 146.9651 86.699) (end 150.35 90.0839) (width 0.2) (layer "F.Cu") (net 1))
 (segment (start 157.125 105.49314) (end 145.7865 94.15464) (width 0.2) (layer "F.Cu") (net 1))
 (segment (start 146.0849 86.699) (end 146.9651 86.699) (width 0.2) (layer "F.Cu") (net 1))
 (segment (start 162.949 94.749) (end 163 94.749) (width 0.2) (layer "F.Cu") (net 10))
 (segment (start 163 94.749) (end 163 90.5) (width 0.2) (layer "F.Cu") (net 10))
 (segment (start 148.646 93.646) (end 148.454 93.646) (width 0.2) (layer "F.Cu") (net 10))
 (segment (start 163 97.701) (end 162.949 97.701) (width 0.2) (layer "F.Cu") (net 10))
 (segment (start 157.951 90.5) (end 153.951 94.5) (width 0.2) (layer "F.Cu") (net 10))
 (segment (start 153.951 96.101) (end 149.349 96.101) (width 0.2) (layer "F.Cu") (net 10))
 (segment (start 146.525 91.717) (end 146.525 87.6) (width 0.2) (layer "F.Cu") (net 10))
 (segment (start 149.349 94.349) (end 148.646 93.646) (width 0.2) (layer "F.Cu") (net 10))
 (segment (start 163 90.5) (end 157.951 90.5) (width 0.2) (layer "F.Cu") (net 10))
 (segment (start 153.951 94.5) (end 153.951 96.101) (width 0.2) (layer "F.Cu") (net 10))
 (segment (start 148.454 93.646) (end 146.525 91.717) (width 0.2) (layer "F.Cu") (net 10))
 (segment (start 149.349 96.101) (end 149.349 94.349) (width 0.2) (layer "F.Cu") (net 10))
 (segment (start 163 104.775) (end 163 97.701) (width 0.2) (layer "F.Cu") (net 10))
 (segment (start 161.425 106.35) (end 163 104.775) (width 0.2) (layer "F.Cu") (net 10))
 (segment (start 162.949 97.701) (end 162.949 94.749) (width 0.2) (layer "F.Cu") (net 10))
 (segment (start 131.375 102.65) (end 140.9 102.65) (width 0.2) (layer "F.Cu") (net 59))
 (segment (start 142.5 104.25) (end 142.5 104.75) (width 0.2) (layer "F.Cu") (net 59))
 (segment (start 142.4625 104.7875) (end 142.4625 113.85) (width 0.2) (layer "F.Cu") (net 59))
 (segment (start 141 102.75) (end 141 101.473) (width 0.2) (layer "F.Cu") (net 59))
 (segment (start 143.25 103.927) (end 142.927 104.25) (width 0.2) (layer "F.Cu") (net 59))
 (segment (start 142.927 104.25) (end 142.5 104.25) (width 0.2) (layer "F.Cu") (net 59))
 (segment (start 141.124 101.349) (end 143.099 101.349) (width 0.2) (layer "F.Cu") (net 59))
 (segment (start 140.9 102.65) (end 141 102.75) (width 0.2) (layer "F.Cu") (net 59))
 (segment (start 143.099 101.349) (end 143.25 101.5) (width 0.2) (layer "F.Cu") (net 59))
 (segment (start 141 101.473) (end 141.124 101.349) (width 0.2) (layer "F.Cu") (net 59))
 (segment (start 142.5 104.75) (end 142.4625 104.7875) (width 0.2) (layer "F.Cu") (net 59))
 (segment (start 143.25 101.5) (end 143.25 103.927) (width 0.2) (layer "F.Cu") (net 59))
 (segment (start 132.5 106.304) (end 132.446 106.25) (width 0.2) (layer "F.Cu") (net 48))
 (segment (start 131.525001 109.445) (end 132.525 109.445) (width 0.2) (layer "F.Cu") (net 48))
 (segment (start 132.85 103.151) (end 132.75 103.051) (width 0.2) (layer "F.Cu") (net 48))
 (segment (start 141.674 103.151) (end 132.85 103.151) (width 0.2) (layer "F.Cu") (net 48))
 (segment (start 142.175 102.65) (end 141.674 103.151) (width 0.2) (layer "F.Cu") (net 48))
 (segment (start 132.75 106.25) (end 132.696 106.304) (width 0.2) (layer "F.Cu") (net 48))
 (segment (start 131.25 106.25) (end 131.224 106.276) (width 0.2) (layer "F.Cu") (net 48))
 (segment (start 142.175 102.65) (end 141.775 102.25) (width 0.2) (layer "F.Cu") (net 48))
 (segment (start 131.224 106.276) (end 131.224 109.143999) (width 0.2) (layer "F.Cu") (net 48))
 (segment (start 132.75 103.051) (end 132.75 106.25) (width 0.2) (layer "F.Cu") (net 48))
 (segment (start 132.696 106.304) (end 132.5 106.304) (width 0.2) (layer "F.Cu") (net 48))
 (segment (start 131.224 109.143999) (end 131.525001 109.445) (width 0.2) (layer "F.Cu") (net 48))
 (segment (start 132.446 106.25) (end 131.25 106.25) (width 0.2) (layer "F.Cu") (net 48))
 (segment (start 139.2375 112.5) (end 140.5875 113.85) (width 0.2) (layer "F.Cu") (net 46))
 (segment (start 139 112.5) (end 139.2375 112.5) (width 0.2) (layer "F.Cu") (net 46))
 (segment (start 138.914 112.586) (end 139 112.5) (width 0.2) (layer "F.Cu") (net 46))
 (segment (start 135.883032 111.985) (end 136.484032 112.586) (width 0.2) (layer "F.Cu") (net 46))
 (segment (start 136.484032 112.586) (end 138.914 112.586) (width 0.2) (layer "F.Cu") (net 46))
 (segment (start 132.525 106.905) (end 135.883032 106.905) (width 0.2) (layer "F.Cu") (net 46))
 (segment (start 135.883032 106.905) (end 135.883032 111.985) (width 0.2) (layer "F.Cu") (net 46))
 (segment (start 157.125 108.35) (end 158.9625 110.1875) (width 0.2) (layer "F.Cu") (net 5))
 (segment (start 158.9625 113.0375) (end 159 113) (width 0.2) (layer "F.Cu") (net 5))
 (segment (start 158.9625 113.0375) (end 158.9625 113.1) (width 0.2) (layer "F.Cu") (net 5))
 (segment (start 158.9625 110.1875) (end 158.9625 113.1) (width 0.2) (layer "F.Cu") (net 5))
 (segment (start 156.299076 106.85) (end 155.965176 107.1839) (width 0.2) (layer "F.Cu") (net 2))
 (segment (start 157.883824 106.85) (end 157.125 106.85) (width 0.2) (layer "F.Cu") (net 2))
 (segment (start 157.901 111.08984) (end 157.901 114.86216) (width 0.2) (layer "F.Cu") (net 2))
 (segment (start 155.965176 107.1839) (end 155.965176 109.154016) (width 0.2) (layer "F.Cu") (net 2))
 (segment (start 157.901 114.86216) (end 158.53884 115.5) (width 0.2) (layer "F.Cu") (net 2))
 (segment (start 159.5 115.5) (end 161.3375 113.6625) (width 0.2) (layer "F.Cu") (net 2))
 (segment (start 157.125 106.85) (end 156.299076 106.85) (width 0.2) (layer "F.Cu") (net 2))
 (segment (start 161.3375 113.1) (end 161.3375 111.7395) (width 0.2) (layer "F.Cu") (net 2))
 (segment (start 161.3375 113.6625) (end 161.3375 113.1) (width 0.2) (layer "F.Cu") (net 2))
 (segment (start 155.965176 109.154016) (end 157.901 111.08984) (width 0.2) (layer "F.Cu") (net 2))
 (segment (start 158.53884 115.5) (end 159.5 115.5) (width 0.2) (layer "F.Cu") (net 2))
 (segment (start 132 117.599) (end 132 116.32) (width 0.2) (layer "F.Cu") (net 25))
 (segment (start 132 116.32) (end 132.525 115.795) (width 0.2) (layer "F.Cu") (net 25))
 (segment (start 150.75 115.35) (end 150.75 115.924999) (width 0.2) (layer "F.Cu") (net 25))
 (segment (start 150.75 115.924999) (end 149.075999 117.599) (width 0.2) (layer "F.Cu") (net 25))
 (segment (start 149.075999 117.599) (end 132 117.599) (width 0.2) (layer "F.Cu") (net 25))
 (segment (start 148.75 115.924999) (end 148.278999 116.396) (width 0.2) (layer "F.Cu") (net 23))
 (segment (start 135.395999 116.396) (end 133.524999 114.525) (width 0.2) (layer "F.Cu") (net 23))
 (segment (start 148.75 115.35) (end 148.75 115.924999) (width 0.2) (layer "F.Cu") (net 23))
 (segment (start 133.524999 114.525) (end 132.525 114.525) (width 0.2) (layer "F.Cu") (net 23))
 (segment (start 148.278999 116.396) (end 135.395999 116.396) (width 0.2) (layer "F.Cu") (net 23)))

